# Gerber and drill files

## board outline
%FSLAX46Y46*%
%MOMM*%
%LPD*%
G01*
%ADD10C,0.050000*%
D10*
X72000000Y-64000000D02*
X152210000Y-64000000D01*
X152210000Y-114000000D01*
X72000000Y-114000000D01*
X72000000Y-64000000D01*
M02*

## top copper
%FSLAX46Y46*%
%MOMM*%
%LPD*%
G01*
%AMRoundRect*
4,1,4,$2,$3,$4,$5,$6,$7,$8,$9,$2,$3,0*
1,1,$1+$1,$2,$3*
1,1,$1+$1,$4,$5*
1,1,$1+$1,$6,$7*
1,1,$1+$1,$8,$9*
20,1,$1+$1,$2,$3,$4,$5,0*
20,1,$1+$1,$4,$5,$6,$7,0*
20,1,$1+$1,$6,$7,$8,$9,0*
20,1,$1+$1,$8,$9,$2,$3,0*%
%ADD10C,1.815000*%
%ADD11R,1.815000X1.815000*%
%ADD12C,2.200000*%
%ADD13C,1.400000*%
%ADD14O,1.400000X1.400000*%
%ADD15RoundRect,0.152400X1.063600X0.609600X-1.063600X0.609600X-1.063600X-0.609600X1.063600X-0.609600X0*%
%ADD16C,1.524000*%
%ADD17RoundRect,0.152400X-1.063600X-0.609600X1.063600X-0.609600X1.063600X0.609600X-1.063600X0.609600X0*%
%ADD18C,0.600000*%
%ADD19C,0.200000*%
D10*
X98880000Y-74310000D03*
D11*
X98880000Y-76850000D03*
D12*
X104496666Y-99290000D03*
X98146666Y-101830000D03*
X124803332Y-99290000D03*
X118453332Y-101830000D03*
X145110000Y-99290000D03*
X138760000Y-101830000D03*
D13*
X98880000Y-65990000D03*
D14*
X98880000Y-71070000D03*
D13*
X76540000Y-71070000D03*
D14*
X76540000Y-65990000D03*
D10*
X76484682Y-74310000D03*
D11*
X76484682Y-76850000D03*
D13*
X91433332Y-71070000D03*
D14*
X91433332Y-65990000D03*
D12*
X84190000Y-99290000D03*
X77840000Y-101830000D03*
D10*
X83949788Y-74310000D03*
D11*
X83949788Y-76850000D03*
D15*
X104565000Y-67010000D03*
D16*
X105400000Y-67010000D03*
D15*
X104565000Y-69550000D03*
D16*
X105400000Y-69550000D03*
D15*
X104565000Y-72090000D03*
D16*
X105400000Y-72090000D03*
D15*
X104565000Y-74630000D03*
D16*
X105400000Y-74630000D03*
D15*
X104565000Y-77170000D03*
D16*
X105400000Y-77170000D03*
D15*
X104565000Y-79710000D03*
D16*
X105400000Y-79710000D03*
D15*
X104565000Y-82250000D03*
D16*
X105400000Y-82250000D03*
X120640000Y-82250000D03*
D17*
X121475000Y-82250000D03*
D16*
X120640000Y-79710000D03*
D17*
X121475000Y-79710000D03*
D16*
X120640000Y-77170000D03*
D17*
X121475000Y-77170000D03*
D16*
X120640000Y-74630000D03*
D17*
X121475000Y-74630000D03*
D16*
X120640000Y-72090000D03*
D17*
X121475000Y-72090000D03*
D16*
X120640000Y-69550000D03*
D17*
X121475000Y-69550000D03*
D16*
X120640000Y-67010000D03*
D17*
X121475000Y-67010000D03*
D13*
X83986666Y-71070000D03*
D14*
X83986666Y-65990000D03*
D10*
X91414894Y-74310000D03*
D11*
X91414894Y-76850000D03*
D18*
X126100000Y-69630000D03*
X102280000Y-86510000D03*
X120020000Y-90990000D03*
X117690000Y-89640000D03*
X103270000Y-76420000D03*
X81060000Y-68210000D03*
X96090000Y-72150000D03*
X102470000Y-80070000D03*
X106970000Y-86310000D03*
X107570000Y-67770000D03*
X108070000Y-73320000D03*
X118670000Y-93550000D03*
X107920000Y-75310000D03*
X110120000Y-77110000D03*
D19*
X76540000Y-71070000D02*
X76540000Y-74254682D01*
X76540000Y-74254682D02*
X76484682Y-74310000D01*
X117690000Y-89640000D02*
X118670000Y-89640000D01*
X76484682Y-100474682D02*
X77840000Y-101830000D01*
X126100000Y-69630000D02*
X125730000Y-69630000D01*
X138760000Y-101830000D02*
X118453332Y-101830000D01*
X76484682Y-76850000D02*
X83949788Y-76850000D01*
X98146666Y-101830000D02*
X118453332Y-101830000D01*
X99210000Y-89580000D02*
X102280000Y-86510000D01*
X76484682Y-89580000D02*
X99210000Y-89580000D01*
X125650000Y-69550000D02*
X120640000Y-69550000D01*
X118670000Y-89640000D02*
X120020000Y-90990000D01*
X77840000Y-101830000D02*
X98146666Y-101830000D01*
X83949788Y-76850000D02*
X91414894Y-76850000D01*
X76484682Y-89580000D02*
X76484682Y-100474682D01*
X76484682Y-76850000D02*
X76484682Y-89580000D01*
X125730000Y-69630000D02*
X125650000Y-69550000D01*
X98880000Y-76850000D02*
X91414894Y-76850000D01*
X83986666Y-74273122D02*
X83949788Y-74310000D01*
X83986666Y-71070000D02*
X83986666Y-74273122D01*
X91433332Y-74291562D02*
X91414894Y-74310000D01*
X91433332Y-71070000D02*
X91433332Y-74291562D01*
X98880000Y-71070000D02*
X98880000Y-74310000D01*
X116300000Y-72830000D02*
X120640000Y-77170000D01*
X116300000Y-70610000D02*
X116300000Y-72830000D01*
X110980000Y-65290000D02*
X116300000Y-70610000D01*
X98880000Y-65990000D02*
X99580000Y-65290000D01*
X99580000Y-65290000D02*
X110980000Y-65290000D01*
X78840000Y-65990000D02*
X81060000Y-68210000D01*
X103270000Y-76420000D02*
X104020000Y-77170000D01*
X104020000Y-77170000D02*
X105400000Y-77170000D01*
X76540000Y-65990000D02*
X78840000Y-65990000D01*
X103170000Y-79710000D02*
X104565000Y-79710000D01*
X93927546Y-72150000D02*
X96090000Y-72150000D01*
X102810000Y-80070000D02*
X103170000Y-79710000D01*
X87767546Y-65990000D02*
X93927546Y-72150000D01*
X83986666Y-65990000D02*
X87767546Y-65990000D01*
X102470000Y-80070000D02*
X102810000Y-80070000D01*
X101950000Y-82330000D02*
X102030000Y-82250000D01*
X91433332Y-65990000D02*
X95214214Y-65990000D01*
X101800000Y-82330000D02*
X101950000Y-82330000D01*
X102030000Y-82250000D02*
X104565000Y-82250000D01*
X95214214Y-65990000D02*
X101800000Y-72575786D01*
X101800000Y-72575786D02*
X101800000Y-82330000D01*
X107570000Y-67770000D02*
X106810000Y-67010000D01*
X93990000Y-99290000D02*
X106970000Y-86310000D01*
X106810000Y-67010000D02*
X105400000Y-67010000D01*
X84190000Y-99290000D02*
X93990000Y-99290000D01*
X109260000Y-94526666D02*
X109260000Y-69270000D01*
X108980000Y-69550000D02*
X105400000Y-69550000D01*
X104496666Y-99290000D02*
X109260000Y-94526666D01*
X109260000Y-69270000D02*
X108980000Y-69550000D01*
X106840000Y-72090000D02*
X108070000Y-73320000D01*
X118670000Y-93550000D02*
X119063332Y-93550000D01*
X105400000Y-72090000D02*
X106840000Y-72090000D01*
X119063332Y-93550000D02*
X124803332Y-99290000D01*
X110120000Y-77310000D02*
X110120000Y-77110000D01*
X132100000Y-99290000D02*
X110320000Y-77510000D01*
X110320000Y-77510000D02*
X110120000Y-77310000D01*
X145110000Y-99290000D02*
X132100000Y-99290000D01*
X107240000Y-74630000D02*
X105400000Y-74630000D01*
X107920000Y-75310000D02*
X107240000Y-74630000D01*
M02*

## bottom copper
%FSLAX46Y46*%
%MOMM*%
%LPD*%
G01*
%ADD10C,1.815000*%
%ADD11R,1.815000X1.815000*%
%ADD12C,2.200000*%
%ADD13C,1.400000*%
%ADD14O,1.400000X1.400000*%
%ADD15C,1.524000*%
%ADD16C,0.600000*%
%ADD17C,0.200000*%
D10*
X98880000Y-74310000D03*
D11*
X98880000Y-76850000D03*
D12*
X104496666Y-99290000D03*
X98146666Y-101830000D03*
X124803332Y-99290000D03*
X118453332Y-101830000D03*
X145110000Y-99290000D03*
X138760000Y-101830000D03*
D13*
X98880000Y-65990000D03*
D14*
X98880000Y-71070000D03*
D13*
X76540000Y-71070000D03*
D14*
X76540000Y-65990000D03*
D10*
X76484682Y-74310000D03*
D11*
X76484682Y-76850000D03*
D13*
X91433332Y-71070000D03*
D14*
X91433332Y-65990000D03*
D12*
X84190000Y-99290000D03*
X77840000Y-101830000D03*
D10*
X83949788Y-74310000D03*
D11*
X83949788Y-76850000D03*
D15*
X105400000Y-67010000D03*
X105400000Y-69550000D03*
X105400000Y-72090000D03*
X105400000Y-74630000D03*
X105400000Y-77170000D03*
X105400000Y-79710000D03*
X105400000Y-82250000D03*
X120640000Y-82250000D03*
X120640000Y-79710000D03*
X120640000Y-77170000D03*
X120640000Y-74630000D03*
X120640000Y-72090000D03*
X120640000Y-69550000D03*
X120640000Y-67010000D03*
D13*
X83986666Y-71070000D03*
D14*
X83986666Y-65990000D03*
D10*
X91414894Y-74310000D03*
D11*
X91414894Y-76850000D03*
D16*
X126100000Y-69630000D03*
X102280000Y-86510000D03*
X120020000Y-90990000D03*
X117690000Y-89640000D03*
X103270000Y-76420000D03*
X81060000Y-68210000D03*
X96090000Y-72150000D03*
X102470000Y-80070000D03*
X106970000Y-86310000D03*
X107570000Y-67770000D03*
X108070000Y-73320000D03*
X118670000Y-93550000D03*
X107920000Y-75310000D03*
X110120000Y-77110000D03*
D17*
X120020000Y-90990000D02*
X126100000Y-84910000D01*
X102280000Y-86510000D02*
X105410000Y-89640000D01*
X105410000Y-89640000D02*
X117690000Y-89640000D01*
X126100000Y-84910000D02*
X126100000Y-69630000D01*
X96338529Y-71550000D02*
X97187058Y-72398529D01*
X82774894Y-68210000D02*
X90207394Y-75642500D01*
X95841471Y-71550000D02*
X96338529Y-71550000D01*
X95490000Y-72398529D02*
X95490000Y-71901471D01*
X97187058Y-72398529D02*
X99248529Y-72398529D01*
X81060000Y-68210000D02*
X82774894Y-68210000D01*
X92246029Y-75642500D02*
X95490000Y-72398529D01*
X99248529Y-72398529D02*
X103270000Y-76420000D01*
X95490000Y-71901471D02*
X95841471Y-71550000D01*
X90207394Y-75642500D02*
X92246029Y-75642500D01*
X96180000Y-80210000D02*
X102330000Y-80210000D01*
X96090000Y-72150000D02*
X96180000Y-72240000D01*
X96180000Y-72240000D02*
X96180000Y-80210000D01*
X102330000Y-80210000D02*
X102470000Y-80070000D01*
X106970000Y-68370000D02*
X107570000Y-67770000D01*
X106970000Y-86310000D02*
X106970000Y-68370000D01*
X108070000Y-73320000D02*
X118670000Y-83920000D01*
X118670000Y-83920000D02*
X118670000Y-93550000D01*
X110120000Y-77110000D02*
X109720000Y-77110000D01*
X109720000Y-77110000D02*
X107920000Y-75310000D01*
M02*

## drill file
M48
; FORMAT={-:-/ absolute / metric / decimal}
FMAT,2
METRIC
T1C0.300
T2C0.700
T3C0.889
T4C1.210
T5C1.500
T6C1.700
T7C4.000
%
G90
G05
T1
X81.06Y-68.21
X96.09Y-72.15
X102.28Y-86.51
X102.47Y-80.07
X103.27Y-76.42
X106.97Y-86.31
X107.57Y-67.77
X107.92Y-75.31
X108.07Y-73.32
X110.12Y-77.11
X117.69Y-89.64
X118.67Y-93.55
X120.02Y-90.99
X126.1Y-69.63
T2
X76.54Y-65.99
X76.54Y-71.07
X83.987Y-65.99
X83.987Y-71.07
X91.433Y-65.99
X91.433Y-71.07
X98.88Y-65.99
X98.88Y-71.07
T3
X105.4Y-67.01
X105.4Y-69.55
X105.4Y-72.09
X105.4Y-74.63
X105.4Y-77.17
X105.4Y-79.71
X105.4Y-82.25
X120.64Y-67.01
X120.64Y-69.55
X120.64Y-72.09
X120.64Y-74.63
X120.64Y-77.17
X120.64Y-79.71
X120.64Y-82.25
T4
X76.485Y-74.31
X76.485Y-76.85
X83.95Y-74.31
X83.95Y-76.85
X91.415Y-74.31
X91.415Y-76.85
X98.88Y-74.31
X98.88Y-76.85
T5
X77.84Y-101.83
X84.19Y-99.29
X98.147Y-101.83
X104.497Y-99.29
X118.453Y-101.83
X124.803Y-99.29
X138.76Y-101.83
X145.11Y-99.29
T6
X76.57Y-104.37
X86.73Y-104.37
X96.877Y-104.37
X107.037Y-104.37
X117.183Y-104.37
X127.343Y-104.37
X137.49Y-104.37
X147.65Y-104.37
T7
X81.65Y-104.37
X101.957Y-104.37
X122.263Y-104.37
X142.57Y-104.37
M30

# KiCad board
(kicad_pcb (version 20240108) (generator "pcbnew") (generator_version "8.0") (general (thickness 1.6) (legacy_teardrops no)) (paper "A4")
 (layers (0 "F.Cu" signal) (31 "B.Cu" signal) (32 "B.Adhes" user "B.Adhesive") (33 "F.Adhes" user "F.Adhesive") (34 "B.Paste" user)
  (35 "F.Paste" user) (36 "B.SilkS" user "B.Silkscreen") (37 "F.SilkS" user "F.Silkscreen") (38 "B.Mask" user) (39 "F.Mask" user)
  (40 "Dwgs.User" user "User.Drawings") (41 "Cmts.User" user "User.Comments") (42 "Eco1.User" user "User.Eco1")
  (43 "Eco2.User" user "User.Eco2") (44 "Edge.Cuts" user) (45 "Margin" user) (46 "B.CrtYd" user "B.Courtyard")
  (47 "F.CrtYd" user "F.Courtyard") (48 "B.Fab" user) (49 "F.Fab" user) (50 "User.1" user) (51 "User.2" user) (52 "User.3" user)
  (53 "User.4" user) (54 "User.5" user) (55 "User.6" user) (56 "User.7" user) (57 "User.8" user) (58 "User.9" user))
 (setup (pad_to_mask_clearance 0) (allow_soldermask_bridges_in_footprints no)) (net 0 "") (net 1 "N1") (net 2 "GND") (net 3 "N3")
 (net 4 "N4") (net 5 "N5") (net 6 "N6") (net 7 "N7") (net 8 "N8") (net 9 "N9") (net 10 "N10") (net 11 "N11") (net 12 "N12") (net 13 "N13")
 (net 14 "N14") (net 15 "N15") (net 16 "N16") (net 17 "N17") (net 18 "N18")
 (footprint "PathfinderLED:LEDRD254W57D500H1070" (layer "F.Cu") (at 98.88 75.58 90)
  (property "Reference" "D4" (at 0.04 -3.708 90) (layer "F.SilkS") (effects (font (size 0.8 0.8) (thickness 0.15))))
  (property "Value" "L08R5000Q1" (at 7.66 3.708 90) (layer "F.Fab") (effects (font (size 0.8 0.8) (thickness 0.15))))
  (pad "A" thru_hole circle (at 1.27 0 90) (size 1.815 1.815) (drill 1.21) (layers "*.Cu" "*.Mask") (remove_unused_layers no) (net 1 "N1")
   (solder_mask_margin 0.102))
  (pad "C" thru_hole rect (at -1.27 0 90) (size 1.815 1.815) (drill 1.21) (layers "*.Cu" "*.Mask") (remove_unused_layers no) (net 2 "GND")
   (solder_mask_margin 0.102)))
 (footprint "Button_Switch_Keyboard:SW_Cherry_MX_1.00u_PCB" (layer "F.Cu") (at 104.496666 99.29)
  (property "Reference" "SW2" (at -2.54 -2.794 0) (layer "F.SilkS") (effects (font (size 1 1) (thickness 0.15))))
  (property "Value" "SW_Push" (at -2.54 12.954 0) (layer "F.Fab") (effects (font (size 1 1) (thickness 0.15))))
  (pad "" np_thru_hole circle (at -7.62 5.08) (size 1.7 1.7) (drill 1.7) (layers "*.Cu" "*.Mask"))
  (pad "" np_thru_hole circle (at -2.54 5.08) (size 4 4) (drill 4) (layers "*.Cu" "*.Mask"))
  (pad "" np_thru_hole circle (at 2.54 5.08) (size 1.7 1.7) (drill 1.7) (layers "*.Cu" "*.Mask"))
  (pad "1" thru_hole circle (at 0 0) (size 2.2 2.2) (drill 1.5) (layers "*.Cu" "*.Mask") (remove_unused_layers no) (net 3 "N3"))
  (pad "2" thru_hole circle (at -6.35 2.54) (size 2.2 2.2) (drill 1.5) (layers "*.Cu" "*.Mask") (remove_unused_layers no) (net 2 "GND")))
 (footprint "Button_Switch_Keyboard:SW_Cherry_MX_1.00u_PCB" (layer "F.Cu") (at 124.803332 99.29)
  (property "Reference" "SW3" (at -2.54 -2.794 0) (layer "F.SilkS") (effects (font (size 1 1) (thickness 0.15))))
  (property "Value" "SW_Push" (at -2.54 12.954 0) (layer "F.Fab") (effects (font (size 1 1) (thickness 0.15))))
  (pad "" np_thru_hole circle (at -7.62 5.08) (size 1.7 1.7) (drill 1.7) (layers "*.Cu" "*.Mask"))
  (pad "" np_thru_hole circle (at -2.54 5.08) (size 4 4) (drill 4) (layers "*.Cu" "*.Mask"))
  (pad "" np_thru_hole circle (at 2.54 5.08) (size 1.7 1.7) (drill 1.7) (layers "*.Cu" "*.Mask"))
  (pad "1" thru_hole circle (at 0 0) (size 2.2 2.2) (drill 1.5) (layers "*.Cu" "*.Mask") (remove_unused_layers no) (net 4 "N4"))
  (pad "2" thru_hole circle (at -6.35 2.54) (size 2.2 2.2) (drill 1.5) (layers "*.Cu" "*.Mask") (remove_unused_layers no) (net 2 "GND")))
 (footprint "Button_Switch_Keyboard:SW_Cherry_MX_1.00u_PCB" (layer "F.Cu") (at 145.11 99.29)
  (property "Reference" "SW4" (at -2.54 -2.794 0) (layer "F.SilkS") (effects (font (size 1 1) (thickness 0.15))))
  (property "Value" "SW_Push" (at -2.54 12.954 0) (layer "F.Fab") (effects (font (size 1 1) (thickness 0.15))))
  (pad "" np_thru_hole circle (at -7.62 5.08) (size 1.7 1.7) (drill 1.7) (layers "*.Cu" "*.Mask"))
  (pad "" np_thru_hole circle (at -2.54 5.08) (size 4 4) (drill 4) (layers "*.Cu" "*.Mask"))
  (pad "" np_thru_hole circle (at 2.54 5.08) (size 1.7 1.7) (drill 1.7) (layers "*.Cu" "*.Mask"))
  (pad "1" thru_hole circle (at 0 0) (size 2.2 2.2) (drill 1.5) (layers "*.Cu" "*.Mask") (remove_unused_layers no) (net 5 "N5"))
  (pad "2" thru_hole circle (at -6.35 2.54) (size 2.2 2.2) (drill 1.5) (layers "*.Cu" "*.Mask") (remove_unused_layers no) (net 2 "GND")))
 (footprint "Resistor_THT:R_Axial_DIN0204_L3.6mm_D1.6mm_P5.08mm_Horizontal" (layer "F.Cu") (at 98.88 65.99 -90)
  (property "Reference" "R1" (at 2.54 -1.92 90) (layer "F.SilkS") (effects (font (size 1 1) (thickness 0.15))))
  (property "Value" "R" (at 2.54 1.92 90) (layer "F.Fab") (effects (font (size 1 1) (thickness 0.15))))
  (pad "1" thru_hole circle (at 0 0 270) (size 1.4 1.4) (drill 0.7) (layers "*.Cu" "*.Mask") (remove_unused_layers no) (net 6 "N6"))
  (pad "2" thru_hole oval (at 5.08 0 270) (size 1.4 1.4) (drill 0.7) (layers "*.Cu" "*.Mask") (remove_unused_layers no) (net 1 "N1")))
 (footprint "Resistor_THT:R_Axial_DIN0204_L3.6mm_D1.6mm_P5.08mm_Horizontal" (layer "F.Cu") (at 76.54 71.07 90)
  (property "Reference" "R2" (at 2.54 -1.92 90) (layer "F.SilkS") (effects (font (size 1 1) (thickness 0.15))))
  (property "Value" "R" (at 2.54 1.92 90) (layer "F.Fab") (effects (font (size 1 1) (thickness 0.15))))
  (pad "1" thru_hole circle (at 0 0 90) (size 1.4 1.4) (drill 0.7) (layers "*.Cu" "*.Mask") (remove_unused_layers no) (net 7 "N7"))
  (pad "2" thru_hole oval (at 5.08 0 90) (size 1.4 1.4) (drill 0.7) (layers "*.Cu" "*.Mask") (remove_unused_layers no) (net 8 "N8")))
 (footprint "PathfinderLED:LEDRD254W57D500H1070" (layer "F.Cu") (at 76.484682 75.58 90)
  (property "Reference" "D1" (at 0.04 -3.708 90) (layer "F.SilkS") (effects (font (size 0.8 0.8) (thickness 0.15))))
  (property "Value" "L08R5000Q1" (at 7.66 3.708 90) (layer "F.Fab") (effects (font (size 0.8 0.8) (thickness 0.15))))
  (pad "A" thru_hole circle (at 1.27 0 90) (size 1.815 1.815) (drill 1.21) (layers "*.Cu" "*.Mask") (remove_unused_layers no) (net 7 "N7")
   (solder_mask_margin 0.102))
  (pad "C" thru_hole rect (at -1.27 0 90) (size 1.815 1.815) (drill 1.21) (layers "*.Cu" "*.Mask") (remove_unused_layers no) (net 2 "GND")
   (solder_mask_margin 0.102)))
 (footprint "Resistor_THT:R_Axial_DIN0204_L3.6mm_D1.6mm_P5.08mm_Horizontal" (layer "F.Cu") (at 91.433332 71.07 90)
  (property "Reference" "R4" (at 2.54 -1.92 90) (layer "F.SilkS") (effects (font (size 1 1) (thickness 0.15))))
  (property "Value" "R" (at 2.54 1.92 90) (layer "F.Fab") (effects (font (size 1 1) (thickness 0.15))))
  (pad "1" thru_hole circle (at 0 0 90) (size 1.4 1.4) (drill 0.7) (layers "*.Cu" "*.Mask") (remove_unused_layers no) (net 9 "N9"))
  (pad "2" thru_hole oval (at 5.08 0 90) (size 1.4 1.4) (drill 0.7) (layers "*.Cu" "*.Mask") (remove_unused_layers no) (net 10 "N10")))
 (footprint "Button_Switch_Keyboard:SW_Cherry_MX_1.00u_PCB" (layer "F.Cu") (at 84.19 99.29)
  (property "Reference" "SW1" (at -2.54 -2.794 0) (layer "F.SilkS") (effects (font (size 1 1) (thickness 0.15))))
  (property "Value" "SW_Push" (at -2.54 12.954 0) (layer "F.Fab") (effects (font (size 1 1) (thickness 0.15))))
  (pad "" np_thru_hole circle (at -7.62 5.08) (size 1.7 1.7) (drill 1.7) (layers "*.Cu" "*.Mask"))
  (pad "" np_thru_hole circle (at -2.54 5.08) (size 4 4) (drill 4) (layers "*.Cu" "*.Mask"))
  (pad "" np_thru_hole circle (at 2.54 5.08) (size 1.7 1.7) (drill 1.7) (layers "*.Cu" "*.Mask"))
  (pad "1" thru_hole circle (at 0 0) (size 2.2 2.2) (drill 1.5) (layers "*.Cu" "*.Mask") (remove_unused_layers no) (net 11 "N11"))
  (pad "2" thru_hole circle (at -6.35 2.54) (size 2.2 2.2) (drill 1.5) (layers "*.Cu" "*.Mask") (remove_unused_layers no) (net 2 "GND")))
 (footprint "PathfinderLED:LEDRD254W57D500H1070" (layer "F.Cu") (at 83.949788 75.58 90)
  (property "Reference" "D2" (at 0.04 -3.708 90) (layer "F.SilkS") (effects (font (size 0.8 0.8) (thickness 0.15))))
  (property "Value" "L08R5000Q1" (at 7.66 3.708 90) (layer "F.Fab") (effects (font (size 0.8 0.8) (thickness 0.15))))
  (pad "A" thru_hole circle (at 1.27 0 90) (size 1.815 1.815) (drill 1.21) (layers "*.Cu" "*.Mask") (remove_unused_layers no) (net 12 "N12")
   (solder_mask_margin 0.102))
  (pad "C" thru_hole rect (at -1.27 0 90) (size 1.815 1.815) (drill 1.21) (layers "*.Cu" "*.Mask") (remove_unused_layers no) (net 2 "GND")
   (solder_mask_margin 0.102)))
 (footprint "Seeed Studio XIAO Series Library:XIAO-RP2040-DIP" (layer "F.Cu") (at 113.02 74.63)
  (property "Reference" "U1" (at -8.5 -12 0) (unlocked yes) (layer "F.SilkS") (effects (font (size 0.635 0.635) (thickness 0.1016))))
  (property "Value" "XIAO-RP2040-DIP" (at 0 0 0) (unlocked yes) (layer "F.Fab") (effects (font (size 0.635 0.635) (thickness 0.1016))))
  (pad "1" smd roundrect (at -8.455 -7.62 180) (size 2.432 1.524) (layers "F.Cu" "F.Mask") (roundrect_rratio 0.1) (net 11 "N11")
   (thermal_bridge_angle 45))
  (pad "1" thru_hole circle (at -7.62 -7.62 180) (size 1.524 1.524) (drill 0.889) (layers "*.Cu" "*.Mask") (remove_unused_layers no)
   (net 11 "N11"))
  (pad "2" smd roundrect (at -8.455 -5.08 180) (size 2.432 1.524) (layers "F.Cu" "F.Mask") (roundrect_rratio 0.1) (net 3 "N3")
   (thermal_bridge_angle 45))
  (pad "2" thru_hole circle (at -7.62 -5.08 180) (size 1.524 1.524) (drill 0.889) (layers "*.Cu" "*.Mask") (remove_unused_layers no)
   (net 3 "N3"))
  (pad "3" smd roundrect (at -8.455 -2.54 180) (size 2.432 1.524) (layers "F.Cu" "F.Mask") (roundrect_rratio 0.1) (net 4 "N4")
   (thermal_bridge_angle 45))
  (pad "3" thru_hole circle (at -7.62 -2.54 180) (size 1.524 1.524) (drill 0.889) (layers "*.Cu" "*.Mask") (remove_unused_layers no)
   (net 4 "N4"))
  (pad "4" smd roundrect (at -8.455 0 180) (size 2.432 1.524) (layers "F.Cu" "F.Mask") (roundrect_rratio 0.1) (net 5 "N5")
   (thermal_bridge_angle 45))
  (pad "4" thru_hole circle (at -7.62 0 180) (size 1.524 1.524) (drill 0.889) (layers "*.Cu" "*.Mask") (remove_unused_layers no)
   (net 5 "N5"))
  (pad "5" smd roundrect (at -8.455 2.54 180) (size 2.432 1.524) (layers "F.Cu" "F.Mask") (roundrect_rratio 0.1) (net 8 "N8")
   (thermal_bridge_angle 45))
  (pad "5" thru_hole circle (at -7.62 2.54 180) (size 1.524 1.524) (drill 0.889) (layers "*.Cu" "*.Mask") (remove_unused_layers no)
   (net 8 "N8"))
  (pad "6" smd roundrect (at -8.455 5.08 180) (size 2.432 1.524) (layers "F.Cu" "F.Mask") (roundrect_rratio 0.1) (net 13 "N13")
   (thermal_bridge_angle 45))
  (pad "6" thru_hole circle (at -7.62 5.08 180) (size 1.524 1.524) (drill 0.889) (layers "*.Cu" "*.Mask") (remove_unused_layers no)
   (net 13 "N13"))
  (pad "7" smd roundrect (at -8.455 7.62 180) (size 2.432 1.524) (layers "F.Cu" "F.Mask") (roundrect_rratio 0.1) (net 10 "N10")
   (thermal_bridge_angle 45))
  (pad "7" thru_hole circle (at -7.62 7.62 180) (size 1.524 1.524) (drill 0.889) (layers "*.Cu" "*.Mask") (remove_unused_layers no)
   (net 10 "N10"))
  (pad "8" thru_hole circle (at 7.62 7.62) (size 1.524 1.524) (drill 0.889) (layers "*.Cu" "*.Mask") (remove_unused_layers no)
   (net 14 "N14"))
  (pad "8" smd roundrect (at 8.455 7.62) (size 2.432 1.524) (layers "F.Cu" "F.Mask") (roundrect_rratio 0.1) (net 14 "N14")
   (thermal_bridge_angle 45))
  (pad "9" thru_hole circle (at 7.62 5.08) (size 1.524 1.524) (drill 0.889) (layers "*.Cu" "*.Mask") (remove_unused_layers no)
   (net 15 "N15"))
  (pad "9" smd roundrect (at 8.455 5.08) (size 2.432 1.524) (layers "F.Cu" "F.Mask") (roundrect_rratio 0.1) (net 15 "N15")
   (thermal_bridge_angle 45))
  (pad "10" thru_hole circle (at 7.62 2.54) (size 1.524 1.524) (drill 0.889) (layers "*.Cu" "*.Mask") (remove_unused_layers no) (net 6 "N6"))
  (pad "10" smd roundrect (at 8.455 2.54) (size 2.432 1.524) (layers "F.Cu" "F.Mask") (roundrect_rratio 0.1) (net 6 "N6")
   (thermal_bridge_angle 45))
  (pad "11" thru_hole circle (at 7.62 0) (size 1.524 1.524) (drill 0.889) (layers "*.Cu" "*.Mask") (remove_unused_layers no) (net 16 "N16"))
  (pad "11" smd roundrect (at 8.455 0) (size 2.432 1.524) (layers "F.Cu" "F.Mask") (roundrect_rratio 0.1) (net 16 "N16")
   (thermal_bridge_angle 45))
  (pad "12" thru_hole circle (at 7.62 -2.54) (size 1.524 1.524) (drill 0.889) (layers "*.Cu" "*.Mask") (remove_unused_layers no)
   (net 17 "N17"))
  (pad "12" smd roundrect (at 8.455 -2.54) (size 2.432 1.524) (layers "F.Cu" "F.Mask") (roundrect_rratio 0.1) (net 17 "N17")
   (thermal_bridge_angle 45))
  (pad "13" thru_hole circle (at 7.62 -5.08) (size 1.524 1.524) (drill 0.889) (layers "*.Cu" "*.Mask") (remove_unused_layers no)
   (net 2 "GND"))
  (pad "13" smd roundrect (at 8.455 -5.08) (size 2.432 1.524) (layers "F.Cu" "F.Mask") (roundrect_rratio 0.1) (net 2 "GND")
   (thermal_bridge_angle 45))
  (pad "14" thru_hole circle (at 7.62 -7.62) (size 1.524 1.524) (drill 0.889) (layers "*.Cu" "*.Mask") (remove_unused_layers no)
   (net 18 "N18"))
  (pad "14" smd roundrect (at 8.455 -7.62) (size 2.432 1.524) (layers "F.Cu" "F.Mask") (roundrect_rratio 0.1) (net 18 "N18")
   (thermal_bridge_angle 45)))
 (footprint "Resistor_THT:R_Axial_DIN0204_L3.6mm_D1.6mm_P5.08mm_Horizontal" (layer "F.Cu") (at 83.986666 71.07 90)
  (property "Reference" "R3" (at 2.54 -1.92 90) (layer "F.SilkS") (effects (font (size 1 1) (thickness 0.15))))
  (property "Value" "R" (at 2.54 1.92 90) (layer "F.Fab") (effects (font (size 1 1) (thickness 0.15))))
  (pad "1" thru_hole circle (at 0 0 90) (size 1.4 1.4) (drill 0.7) (layers "*.Cu" "*.Mask") (remove_unused_layers no) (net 12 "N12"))
  (pad "2" thru_hole oval (at 5.08 0 90) (size 1.4 1.4) (drill 0.7) (layers "*.Cu" "*.Mask") (remove_unused_layers no) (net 13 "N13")))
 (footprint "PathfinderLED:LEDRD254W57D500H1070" (layer "F.Cu") (at 91.414894 75.58 90)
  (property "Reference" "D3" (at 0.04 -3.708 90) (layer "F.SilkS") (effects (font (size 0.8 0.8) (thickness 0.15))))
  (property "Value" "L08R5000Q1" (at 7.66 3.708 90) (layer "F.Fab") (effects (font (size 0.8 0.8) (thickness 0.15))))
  (pad "A" thru_hole circle (at 1.27 0 90) (size 1.815 1.815) (drill 1.21) (layers "*.Cu" "*.Mask") (remove_unused_layers no) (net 9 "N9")
   (solder_mask_margin 0.102))
  (pad "C" thru_hole rect (at -1.27 0 90) (size 1.815 1.815) (drill 1.21) (layers "*.Cu" "*.Mask") (remove_unused_layers no) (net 2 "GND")
   (solder_mask_margin 0.102)))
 (gr_rect (start 72 64) (end 152.21 114) (stroke (width 0.05) (type default)) (fill none) (layer "Edge.Cuts"))
 (segment (start 76.54 71.07) (end 76.54 74.254682) (width 0.2) (layer "F.Cu") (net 7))
 (segment (start 76.54 74.254682) (end 76.484682 74.31) (width 0.2) (layer "F.Cu") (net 7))
 (segment (start 117.69 89.64) (end 118.67 89.64) (width 0.2) (layer "F.Cu") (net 2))
 (segment (start 76.484682 100.474682) (end 77.84 101.83) (width 0.2) (layer "F.Cu") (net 2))
 (segment (start 126.1 69.63) (end 125.73 69.63) (width 0.2) (layer "F.Cu") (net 2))
 (segment (start 138.76 101.83) (end 118.453332 101.83) (width 0.2) (layer "F.Cu") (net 2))
 (segment (start 76.484682 76.85) (end 83.949788 76.85) (width 0.2) (layer "F.Cu") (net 2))
 (segment (start 98.146666 101.83) (end 118.453332 101.83) (width 0.2) (layer "F.Cu") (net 2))
 (segment (start 99.21 89.58) (end 102.28 86.51) (width 0.2) (layer "F.Cu") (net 2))
 (segment (start 76.484682 89.58) (end 99.21 89.58) (width 0.2) (layer "F.Cu") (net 2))
 (segment (start 125.65 69.55) (end 120.64 69.55) (width 0.2) (layer "F.Cu") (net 2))
 (segment (start 118.67 89.64) (end 120.02 90.99) (width 0.2) (layer "F.Cu") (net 2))
 (segment (start 77.84 101.83) (end 98.146666 101.83) (width 0.2) (layer "F.Cu") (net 2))
 (segment (start 83.949788 76.85) (end 91.414894 76.85) (width 0.2) (layer "F.Cu") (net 2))
 (segment (start 76.484682 89.58) (end 76.484682 100.474682) (width 0.2) (layer "F.Cu") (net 2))
 (segment (start 76.484682 76.85) (end 76.484682 89.58) (width 0.2) (layer "F.Cu") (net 2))
 (segment (start 125.73 69.63) (end 125.65 69.55) (width 0.2) (layer "F.Cu") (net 2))
 (segment (start 98.88 76.85) (end 91.414894 76.85) (width 0.2) (layer "F.Cu") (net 2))
 (via (at 126.1 69.63) (size 0.6) (drill 0.3) (layers "F.Cu" "B.Cu") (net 2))
 (via (at 102.28 86.51) (size 0.6) (drill 0.3) (layers "F.Cu" "B.Cu") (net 2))
 (via (at 120.02 90.99) (size 0.6) (drill 0.3) (layers "F.Cu" "B.Cu") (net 2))
 (via (at 117.69 89.64) (size 0.6) (drill 0.3) (layers "F.Cu" "B.Cu") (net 2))
 (segment (start 120.02 90.99) (end 126.1 84.91) (width 0.2) (layer "B.Cu") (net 2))
 (segment (start 102.28 86.51) (end 105.41 89.64) (width 0.2) (layer "B.Cu") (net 2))
 (segment (start 105.41 89.64) (end 117.69 89.64) (width 0.2) (layer "B.Cu") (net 2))
 (segment (start 126.1 84.91) (end 126.1 69.63) (width 0.2) (layer "B.Cu") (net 2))
 (segment (start 83.986666 74.273122) (end 83.949788 74.31) (width 0.2) (layer "F.Cu") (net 12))
 (segment (start 83.986666 71.07) (end 83.986666 74.273122) (width 0.2) (layer "F.Cu") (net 12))
 (segment (start 91.433332 74.291562) (end 91.414894 74.31) (width 0.2) (layer "F.Cu") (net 9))
 (segment (start 91.433332 71.07) (end 91.433332 74.291562) (width 0.2) (layer "F.Cu") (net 9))
 (segment (start 98.88 71.07) (end 98.88 74.31) (width 0.2) (layer "F.Cu") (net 1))
 (segment (start 116.3 72.83) (end 120.64 77.17) (width 0.2) (layer "F.Cu") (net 6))
 (segment (start 116.3 70.61) (end 116.3 72.83) (width 0.2) (layer "F.Cu") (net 6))
 (segment (start 110.98 65.29) (end 116.3 70.61) (width 0.2) (layer "F.Cu") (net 6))
 (segment (start 98.88 65.99) (end 99.58 65.29) (width 0.2) (layer "F.Cu") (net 6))
 (segment (start 99.58 65.29) (end 110.98 65.29) (width 0.2) (layer "F.Cu") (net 6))
 (segment (start 78.84 65.99) (end 81.06 68.21) (width 0.2) (layer "F.Cu") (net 8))
 (segment (start 103.27 76.42) (end 104.02 77.17) (width 0.2) (layer "F.Cu") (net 8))
 (segment (start 104.02 77.17) (end 105.4 77.17) (width 0.2) (layer "F.Cu") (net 8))
 (segment (start 76.54 65.99) (end 78.84 65.99) (width 0.2) (layer "F.Cu") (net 8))
 (via (at 103.27 76.42) (size 0.6) (drill 0.3) (layers "F.Cu" "B.Cu") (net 8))
 (via (at 81.06 68.21) (size 0.6) (drill 0.3) (layers "F.Cu" "B.Cu") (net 8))
 (segment (start 96.338529 71.55) (end 97.187058 72.398529) (width 0.2) (layer "B.Cu") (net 8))
 (segment (start 82.774894 68.21) (end 90.207394 75.6425) (width 0.2) (layer "B.Cu") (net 8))
 (segment (start 95.841471 71.55) (end 96.338529 71.55) (width 0.2) (layer "B.Cu") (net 8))
 (segment (start 95.49 72.398529) (end 95.49 71.901471) (width 0.2) (layer "B.Cu") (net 8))
 (segment (start 97.187058 72.398529) (end 99.248529 72.398529) (width 0.2) (layer "B.Cu") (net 8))
 (segment (start 81.06 68.21) (end 82.774894 68.21) (width 0.2) (layer "B.Cu") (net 8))
 (segment (start 92.246029 75.6425) (end 95.49 72.398529) (width 0.2) (layer "B.Cu") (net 8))
 (segment (start 99.248529 72.398529) (end 103.27 76.42) (width 0.2) (layer "B.Cu") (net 8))
 (segment (start 95.49 71.901471) (end 95.841471 71.55) (width 0.2) (layer "B.Cu") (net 8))
 (segment (start 90.207394 75.6425) (end 92.246029 75.6425) (width 0.2) (layer "B.Cu") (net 8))
 (segment (start 103.17 79.71) (end 104.565 79.71) (width 0.2) (layer "F.Cu") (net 13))
 (segment (start 93.927546 72.15) (end 96.09 72.15) (width 0.2) (layer "F.Cu") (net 13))
 (segment (start 102.81 80.07) (end 103.17 79.71) (width 0.2) (layer "F.Cu") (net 13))
 (segment (start 87.767546 65.99) (end 93.927546 72.15) (width 0.2) (layer "F.Cu") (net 13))
 (segment (start 83.986666 65.99) (end 87.767546 65.99) (width 0.2) (layer "F.Cu") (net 13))
 (segment (start 102.47 80.07) (end 102.81 80.07) (width 0.2) (layer "F.Cu") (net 13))
 (via (at 96.09 72.15) (size 0.6) (drill 0.3) (layers "F.Cu" "B.Cu") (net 13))
 (via (at 102.47 80.07) (size 0.6) (drill 0.3) (layers "F.Cu" "B.Cu") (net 13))
 (segment (start 96.18 80.21) (end 102.33 80.21) (width 0.2) (layer "B.Cu") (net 13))
 (segment (start 96.09 72.15) (end 96.18 72.24) (width 0.2) (layer "B.Cu") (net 13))
 (segment (start 96.18 72.24) (end 96.18 80.21) (width 0.2) (layer "B.Cu") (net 13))
 (segment (start 102.33 80.21) (end 102.47 80.07) (width 0.2) (layer "B.Cu") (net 13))
 (segment (start 101.95 82.33) (end 102.03 82.25) (width 0.2) (layer "F.Cu") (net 10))
 (segment (start 91.433332 65.99) (end 95.214214 65.99) (width 0.2) (layer "F.Cu") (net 10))
 (segment (start 101.8 82.33) (end 101.95 82.33) (width 0.2) (layer "F.Cu") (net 10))
 (segment (start 102.03 82.25) (end 104.565 82.25) (width 0.2) (layer "F.Cu") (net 10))
 (segment (start 95.214214 65.99) (end 101.8 72.575786) (width 0.2) (layer "F.Cu") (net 10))
 (segment (start 101.8 72.575786) (end 101.8 82.33) (width 0.2) (layer "F.Cu") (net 10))
 (segment (start 107.57 67.77) (end 106.81 67.01) (width 0.2) (layer "F.Cu") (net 11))
 (segment (start 93.99 99.29) (end 106.97 86.31) (width 0.2) (layer "F.Cu") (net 11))
 (segment (start 106.81 67.01) (end 105.4 67.01) (width 0.2) (layer "F.Cu") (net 11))
 (segment (start 84.19 99.29) (end 93.99 99.29) (width 0.2) (layer "F.Cu") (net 11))
 (via (at 106.97 86.31) (size 0.6) (drill 0.3) (layers "F.Cu" "B.Cu") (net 11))
 (via (at 107.57 67.77) (size 0.6) (drill 0.3) (layers "F.Cu" "B.Cu") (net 11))
 (segment (start 106.97 68.37) (end 107.57 67.77) (width 0.2) (layer "B.Cu") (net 11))
 (segment (start 106.97 86.31) (end 106.97 68.37) (width 0.2) (layer "B.Cu") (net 11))
 (segment (start 109.26 94.526666) (end 109.26 69.27) (width 0.2) (layer "F.Cu") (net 3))
 (segment (start 108.98 69.55) (end 105.4 69.55) (width 0.2) (layer "F.Cu") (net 3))
 (segment (start 104.496666 99.29) (end 109.26 94.526666) (width 0.2) (layer "F.Cu") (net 3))
 (segment (start 109.26 69.27) (end 108.98 69.55) (width 0.2) (layer "F.Cu") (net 3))
 (segment (start 106.84 72.09) (end 108.07 73.32) (width 0.2) (layer "F.Cu") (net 4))
 (segment (start 118.67 93.55) (end 119.063332 93.55) (width 0.2) (layer "F.Cu") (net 4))
 (segment (start 105.4 72.09) (end 106.84 72.09) (width 0.2) (layer "F.Cu") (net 4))
 (segment (start 119.063332 93.55) (end 124.803332 99.29) (width 0.2) (layer "F.Cu") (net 4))
 (via (at 108.07 73.32) (size 0.6) (drill 0.3) (layers "F.Cu" "B.Cu") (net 4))
 (via (at 118.67 93.55) (size 0.6) (drill 0.3) (layers "F.Cu" "B.Cu") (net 4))
 (segment (start 108.07 73.32) (end 118.67 83.92) (width 0.2) (layer "B.Cu") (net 4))
 (segment (start 118.67 83.92) (end 118.67 93.55) (width 0.2) (layer "B.Cu") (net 4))
 (segment (start 110.12 77.31) (end 110.12 77.11) (width 0.2) (layer "F.Cu") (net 5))
 (segment (start 132.1 99.29) (end 110.32 77.51) (width 0.2) (layer "F.Cu") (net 5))
 (segment (start 110.32 77.51) (end 110.12 77.31) (width 0.2) (layer "F.Cu") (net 5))
 (segment (start 145.11 99.29) (end 132.1 99.29) (width 0.2) (layer "F.Cu") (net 5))
 (segment (start 107.24 74.63) (end 105.4 74.63) (width 0.2) (layer "F.Cu") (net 5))
 (segment (start 107.92 75.31) (end 107.24 74.63) (width 0.2) (layer "F.Cu") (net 5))
 (via (at 107.92 75.31) (size 0.6) (drill 0.3) (layers "F.Cu" "B.Cu") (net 5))
 (via (at 110.12 77.11) (size 0.6) (drill 0.3) (layers "F.Cu" "B.Cu") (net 5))
 (segment (start 110.12 77.11) (end 109.72 77.11) (width 0.2) (layer "B.Cu") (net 5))
 (segment (start 109.72 77.11) (end 107.92 75.31) (width 0.2) (layer "B.Cu") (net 5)))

